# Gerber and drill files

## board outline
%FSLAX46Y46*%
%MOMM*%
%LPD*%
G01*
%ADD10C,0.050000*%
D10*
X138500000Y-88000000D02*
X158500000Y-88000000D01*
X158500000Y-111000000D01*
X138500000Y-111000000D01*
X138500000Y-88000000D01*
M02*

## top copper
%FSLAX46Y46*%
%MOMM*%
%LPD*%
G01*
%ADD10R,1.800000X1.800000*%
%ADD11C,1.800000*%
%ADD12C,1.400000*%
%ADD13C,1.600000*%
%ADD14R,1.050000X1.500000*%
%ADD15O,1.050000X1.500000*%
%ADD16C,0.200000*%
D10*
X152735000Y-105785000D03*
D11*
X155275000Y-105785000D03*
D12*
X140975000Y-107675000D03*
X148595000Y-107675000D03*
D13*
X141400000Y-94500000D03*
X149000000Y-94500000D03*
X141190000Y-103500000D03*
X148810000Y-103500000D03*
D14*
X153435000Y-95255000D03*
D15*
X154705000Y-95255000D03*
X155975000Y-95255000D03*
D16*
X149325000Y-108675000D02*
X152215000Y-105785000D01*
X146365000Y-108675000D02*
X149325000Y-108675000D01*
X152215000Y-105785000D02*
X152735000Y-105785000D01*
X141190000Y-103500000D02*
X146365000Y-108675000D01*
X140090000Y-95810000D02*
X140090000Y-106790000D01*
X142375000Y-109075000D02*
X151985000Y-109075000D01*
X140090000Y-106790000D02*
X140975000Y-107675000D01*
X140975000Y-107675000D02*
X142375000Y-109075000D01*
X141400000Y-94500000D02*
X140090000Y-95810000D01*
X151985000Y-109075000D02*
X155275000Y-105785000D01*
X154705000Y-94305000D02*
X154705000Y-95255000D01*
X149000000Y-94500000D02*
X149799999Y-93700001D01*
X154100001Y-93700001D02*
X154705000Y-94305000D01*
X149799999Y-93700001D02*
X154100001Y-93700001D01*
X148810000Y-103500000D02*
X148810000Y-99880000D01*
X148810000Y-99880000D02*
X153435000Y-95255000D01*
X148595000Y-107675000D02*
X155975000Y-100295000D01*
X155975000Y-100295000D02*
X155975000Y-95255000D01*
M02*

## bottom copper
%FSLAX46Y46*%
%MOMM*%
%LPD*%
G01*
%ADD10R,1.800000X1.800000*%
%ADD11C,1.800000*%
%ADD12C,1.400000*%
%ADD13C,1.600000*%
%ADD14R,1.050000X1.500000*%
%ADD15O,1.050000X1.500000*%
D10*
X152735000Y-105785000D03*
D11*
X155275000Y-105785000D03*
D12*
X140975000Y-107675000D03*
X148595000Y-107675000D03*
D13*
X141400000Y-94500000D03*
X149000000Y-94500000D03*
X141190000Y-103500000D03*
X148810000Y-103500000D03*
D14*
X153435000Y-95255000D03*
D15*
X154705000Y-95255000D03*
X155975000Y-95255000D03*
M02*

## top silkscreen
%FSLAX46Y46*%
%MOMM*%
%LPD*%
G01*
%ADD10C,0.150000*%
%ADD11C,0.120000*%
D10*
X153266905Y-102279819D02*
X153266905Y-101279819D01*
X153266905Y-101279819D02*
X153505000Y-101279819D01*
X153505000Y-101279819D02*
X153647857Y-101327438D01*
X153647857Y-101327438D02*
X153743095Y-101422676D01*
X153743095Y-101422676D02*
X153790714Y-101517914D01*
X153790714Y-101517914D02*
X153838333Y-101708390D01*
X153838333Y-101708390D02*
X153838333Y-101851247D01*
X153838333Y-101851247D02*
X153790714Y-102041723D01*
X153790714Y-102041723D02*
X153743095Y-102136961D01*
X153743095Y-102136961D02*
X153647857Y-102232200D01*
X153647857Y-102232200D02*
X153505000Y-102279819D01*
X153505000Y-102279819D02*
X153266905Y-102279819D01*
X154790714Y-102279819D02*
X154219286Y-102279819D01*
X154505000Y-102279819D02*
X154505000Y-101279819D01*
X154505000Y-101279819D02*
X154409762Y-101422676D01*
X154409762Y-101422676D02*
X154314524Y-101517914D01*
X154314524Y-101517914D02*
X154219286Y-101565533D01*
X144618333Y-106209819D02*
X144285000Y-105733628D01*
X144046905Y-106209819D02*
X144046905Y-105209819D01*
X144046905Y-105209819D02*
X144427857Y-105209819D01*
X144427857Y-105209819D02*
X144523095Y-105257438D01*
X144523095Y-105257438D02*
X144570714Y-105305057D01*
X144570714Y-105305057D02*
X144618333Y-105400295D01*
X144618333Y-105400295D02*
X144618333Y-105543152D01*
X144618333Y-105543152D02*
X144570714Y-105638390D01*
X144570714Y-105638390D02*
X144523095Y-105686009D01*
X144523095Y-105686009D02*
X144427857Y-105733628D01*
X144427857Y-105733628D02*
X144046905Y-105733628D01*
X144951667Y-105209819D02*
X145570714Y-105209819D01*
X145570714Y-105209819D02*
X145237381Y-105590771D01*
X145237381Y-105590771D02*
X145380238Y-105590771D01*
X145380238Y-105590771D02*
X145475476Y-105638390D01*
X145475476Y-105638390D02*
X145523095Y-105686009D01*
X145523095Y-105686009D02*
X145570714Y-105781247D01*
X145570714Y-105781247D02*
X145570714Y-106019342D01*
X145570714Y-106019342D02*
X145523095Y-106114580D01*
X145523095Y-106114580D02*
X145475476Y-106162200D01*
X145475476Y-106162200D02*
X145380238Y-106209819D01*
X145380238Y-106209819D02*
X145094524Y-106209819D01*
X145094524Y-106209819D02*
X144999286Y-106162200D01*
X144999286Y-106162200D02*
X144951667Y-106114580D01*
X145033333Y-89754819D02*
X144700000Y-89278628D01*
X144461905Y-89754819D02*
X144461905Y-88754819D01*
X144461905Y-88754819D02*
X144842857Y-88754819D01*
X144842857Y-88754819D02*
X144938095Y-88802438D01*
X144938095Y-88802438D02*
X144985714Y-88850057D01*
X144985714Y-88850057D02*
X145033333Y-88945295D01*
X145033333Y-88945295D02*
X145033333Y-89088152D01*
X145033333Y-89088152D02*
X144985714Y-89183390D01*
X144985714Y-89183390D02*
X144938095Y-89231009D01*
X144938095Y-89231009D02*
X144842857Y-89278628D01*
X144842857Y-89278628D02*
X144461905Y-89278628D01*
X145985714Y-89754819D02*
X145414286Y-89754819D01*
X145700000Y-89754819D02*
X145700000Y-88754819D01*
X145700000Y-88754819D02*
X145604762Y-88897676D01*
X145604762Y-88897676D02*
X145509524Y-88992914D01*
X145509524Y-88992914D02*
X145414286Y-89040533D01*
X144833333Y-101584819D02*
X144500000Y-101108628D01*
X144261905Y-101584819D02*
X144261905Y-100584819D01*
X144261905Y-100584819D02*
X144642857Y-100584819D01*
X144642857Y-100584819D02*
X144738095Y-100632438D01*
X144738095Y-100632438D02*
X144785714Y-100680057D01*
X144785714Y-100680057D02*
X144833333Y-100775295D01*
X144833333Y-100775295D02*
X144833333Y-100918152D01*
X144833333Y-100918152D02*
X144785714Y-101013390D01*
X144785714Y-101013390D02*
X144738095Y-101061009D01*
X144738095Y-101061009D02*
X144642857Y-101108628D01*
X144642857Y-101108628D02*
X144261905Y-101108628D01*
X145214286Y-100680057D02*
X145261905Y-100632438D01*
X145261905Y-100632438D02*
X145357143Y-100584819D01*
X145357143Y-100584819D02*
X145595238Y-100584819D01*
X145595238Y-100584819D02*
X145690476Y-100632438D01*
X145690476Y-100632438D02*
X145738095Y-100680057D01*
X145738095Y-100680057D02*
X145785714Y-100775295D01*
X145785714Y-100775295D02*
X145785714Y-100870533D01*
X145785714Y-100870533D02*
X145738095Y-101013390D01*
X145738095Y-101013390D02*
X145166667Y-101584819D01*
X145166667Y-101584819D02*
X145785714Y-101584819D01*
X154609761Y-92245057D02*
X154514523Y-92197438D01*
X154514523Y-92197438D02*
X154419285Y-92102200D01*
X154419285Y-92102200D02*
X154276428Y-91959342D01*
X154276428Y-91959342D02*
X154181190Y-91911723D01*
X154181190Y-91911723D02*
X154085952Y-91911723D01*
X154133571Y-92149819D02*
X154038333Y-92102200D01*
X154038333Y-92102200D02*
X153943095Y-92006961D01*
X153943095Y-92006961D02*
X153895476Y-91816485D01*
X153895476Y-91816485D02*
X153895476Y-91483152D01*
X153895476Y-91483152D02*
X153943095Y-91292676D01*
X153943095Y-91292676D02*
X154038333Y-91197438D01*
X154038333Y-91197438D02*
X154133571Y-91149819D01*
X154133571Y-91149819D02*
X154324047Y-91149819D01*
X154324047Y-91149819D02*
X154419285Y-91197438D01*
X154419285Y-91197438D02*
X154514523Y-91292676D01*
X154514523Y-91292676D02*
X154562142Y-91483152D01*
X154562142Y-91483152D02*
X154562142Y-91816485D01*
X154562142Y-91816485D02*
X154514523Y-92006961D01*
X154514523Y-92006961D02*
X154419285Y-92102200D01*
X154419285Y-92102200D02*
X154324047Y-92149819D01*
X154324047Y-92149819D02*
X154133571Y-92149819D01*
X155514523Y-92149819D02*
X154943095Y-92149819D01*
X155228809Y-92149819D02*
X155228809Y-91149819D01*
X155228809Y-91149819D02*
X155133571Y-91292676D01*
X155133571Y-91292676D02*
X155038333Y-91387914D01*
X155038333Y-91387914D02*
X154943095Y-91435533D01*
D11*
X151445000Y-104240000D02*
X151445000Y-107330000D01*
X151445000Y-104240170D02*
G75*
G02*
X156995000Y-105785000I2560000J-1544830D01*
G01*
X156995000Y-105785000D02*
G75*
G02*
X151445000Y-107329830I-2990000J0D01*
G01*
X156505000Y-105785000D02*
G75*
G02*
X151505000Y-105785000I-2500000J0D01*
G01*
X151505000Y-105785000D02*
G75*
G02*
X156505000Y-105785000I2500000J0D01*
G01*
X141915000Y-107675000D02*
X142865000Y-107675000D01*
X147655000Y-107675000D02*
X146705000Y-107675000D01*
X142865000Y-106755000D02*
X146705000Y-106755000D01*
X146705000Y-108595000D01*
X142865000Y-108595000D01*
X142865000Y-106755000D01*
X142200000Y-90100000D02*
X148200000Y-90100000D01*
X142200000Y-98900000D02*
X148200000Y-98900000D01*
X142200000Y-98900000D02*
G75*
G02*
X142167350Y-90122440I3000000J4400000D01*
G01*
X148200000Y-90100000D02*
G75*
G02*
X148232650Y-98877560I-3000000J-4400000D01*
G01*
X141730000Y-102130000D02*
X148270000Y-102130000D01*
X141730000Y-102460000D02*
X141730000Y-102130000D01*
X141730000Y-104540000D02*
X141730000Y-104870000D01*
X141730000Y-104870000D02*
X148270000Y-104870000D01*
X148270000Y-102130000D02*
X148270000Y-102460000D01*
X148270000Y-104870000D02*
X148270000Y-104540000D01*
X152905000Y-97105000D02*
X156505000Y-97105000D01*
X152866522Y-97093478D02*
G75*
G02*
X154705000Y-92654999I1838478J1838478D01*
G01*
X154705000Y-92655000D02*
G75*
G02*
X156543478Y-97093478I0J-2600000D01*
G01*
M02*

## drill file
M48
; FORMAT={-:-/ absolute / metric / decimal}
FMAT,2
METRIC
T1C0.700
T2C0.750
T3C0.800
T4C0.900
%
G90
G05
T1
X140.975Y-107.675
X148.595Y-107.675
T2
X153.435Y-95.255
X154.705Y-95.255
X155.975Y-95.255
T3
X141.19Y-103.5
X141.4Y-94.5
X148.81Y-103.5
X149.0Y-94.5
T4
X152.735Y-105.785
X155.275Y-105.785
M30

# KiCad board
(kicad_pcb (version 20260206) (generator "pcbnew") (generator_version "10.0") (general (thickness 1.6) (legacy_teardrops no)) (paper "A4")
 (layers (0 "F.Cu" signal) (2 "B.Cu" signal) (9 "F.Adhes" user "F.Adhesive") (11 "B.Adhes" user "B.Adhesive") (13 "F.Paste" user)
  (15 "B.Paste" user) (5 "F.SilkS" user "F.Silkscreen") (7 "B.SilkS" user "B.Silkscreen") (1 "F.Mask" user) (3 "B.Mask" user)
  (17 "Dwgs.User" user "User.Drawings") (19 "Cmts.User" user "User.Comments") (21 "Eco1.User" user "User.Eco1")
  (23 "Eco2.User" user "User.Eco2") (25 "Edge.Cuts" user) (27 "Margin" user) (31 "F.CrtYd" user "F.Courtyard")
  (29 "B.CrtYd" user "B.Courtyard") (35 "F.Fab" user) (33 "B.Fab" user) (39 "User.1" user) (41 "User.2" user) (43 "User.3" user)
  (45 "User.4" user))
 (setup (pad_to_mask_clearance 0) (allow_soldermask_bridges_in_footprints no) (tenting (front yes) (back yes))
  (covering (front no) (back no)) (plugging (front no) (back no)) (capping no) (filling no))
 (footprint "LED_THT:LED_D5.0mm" (layer "F.Cu") (at 152.735 105.785)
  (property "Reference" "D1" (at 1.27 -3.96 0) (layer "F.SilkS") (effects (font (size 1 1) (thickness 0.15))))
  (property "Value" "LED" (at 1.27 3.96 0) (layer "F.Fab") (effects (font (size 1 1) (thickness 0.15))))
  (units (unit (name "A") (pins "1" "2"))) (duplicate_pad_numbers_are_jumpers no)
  (fp_line (start -1.29 -1.545) (end -1.29 1.545) (stroke (width 0.12) (type solid)) (layer "F.SilkS"))
  (fp_arc (start -1.29 -1.54483) (mid 2.071779 -2.880495) (end 4.26 0) (stroke (width 0.12) (type solid)) (layer "F.SilkS"))
  (fp_arc (start 4.26 0) (mid 2.071779 2.880495) (end -1.29 1.54483) (stroke (width 0.12) (type solid)) (layer "F.SilkS"))
  (fp_circle (center 1.27 0) (end 3.77 0) (stroke (width 0.12) (type solid)) (fill no) (layer "F.SilkS"))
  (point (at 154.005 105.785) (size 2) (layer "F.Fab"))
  (pad "1" thru_hole rect (at 0 0) (size 1.8 1.8) (drill 0.9) (layers "*.Cu" "*.Mask") (remove_unused_layers no) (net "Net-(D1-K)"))
  (pad "2" thru_hole circle (at 2.54 0) (size 1.8 1.8) (drill 0.9) (layers "*.Cu" "*.Mask") (remove_unused_layers no) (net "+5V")))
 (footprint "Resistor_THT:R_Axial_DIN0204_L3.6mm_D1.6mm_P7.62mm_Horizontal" (layer "F.Cu") (at 140.975 107.675)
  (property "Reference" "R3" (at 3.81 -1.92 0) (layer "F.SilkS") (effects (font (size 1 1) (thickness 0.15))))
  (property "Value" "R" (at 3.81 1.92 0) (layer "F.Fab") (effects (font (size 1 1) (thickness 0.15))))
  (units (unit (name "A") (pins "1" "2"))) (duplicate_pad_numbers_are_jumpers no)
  (fp_line (start 0.94 0) (end 1.89 0) (stroke (width 0.12) (type solid)) (layer "F.SilkS"))
  (fp_line (start 6.68 0) (end 5.73 0) (stroke (width 0.12) (type solid)) (layer "F.SilkS"))
  (fp_rect (start 1.89 -0.92) (end 5.73 0.92) (stroke (width 0.12) (type solid)) (fill no) (layer "F.SilkS"))
  (pad "1" thru_hole circle (at 0 0) (size 1.4 1.4) (drill 0.7) (layers "*.Cu" "*.Mask") (remove_unused_layers no) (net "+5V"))
  (pad "2" thru_hole circle (at 7.62 0) (size 1.4 1.4) (drill 0.7) (layers "*.Cu" "*.Mask") (remove_unused_layers no) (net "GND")))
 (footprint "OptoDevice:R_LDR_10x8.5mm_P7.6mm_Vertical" (layer "F.Cu") (at 141.4 94.5)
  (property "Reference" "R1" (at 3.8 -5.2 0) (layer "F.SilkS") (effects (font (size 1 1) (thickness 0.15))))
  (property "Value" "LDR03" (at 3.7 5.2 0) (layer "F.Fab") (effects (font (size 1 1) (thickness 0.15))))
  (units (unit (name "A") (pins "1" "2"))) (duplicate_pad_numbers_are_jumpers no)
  (fp_line (start 0.8 -4.4) (end 6.8 -4.4) (stroke (width 0.12) (type solid)) (layer "F.SilkS"))
  (fp_line (start 0.8 4.4) (end 6.8 4.4) (stroke (width 0.12) (type solid)) (layer "F.SilkS"))
  (fp_arc (start 0.8 4.4) (mid -1.525374 0.019809) (end 0.76735 -4.37756) (stroke (width 0.12) (type solid)) (layer "F.SilkS"))
  (fp_arc (start 6.8 -4.4) (mid 9.125374 -0.019809) (end 6.83265 4.37756) (stroke (width 0.12) (type solid)) (layer "F.SilkS"))
  (pad "1" thru_hole circle (at 0 0) (size 1.6 1.6) (drill 0.8) (layers "*.Cu" "*.Mask") (remove_unused_layers no) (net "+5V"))
  (pad "2" thru_hole circle (at 7.6 0) (size 1.6 1.6) (drill 0.8) (layers "*.Cu" "*.Mask") (remove_unused_layers no) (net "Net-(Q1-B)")))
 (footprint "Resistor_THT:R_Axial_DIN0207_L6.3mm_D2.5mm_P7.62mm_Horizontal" (layer "F.Cu") (at 141.19 103.5)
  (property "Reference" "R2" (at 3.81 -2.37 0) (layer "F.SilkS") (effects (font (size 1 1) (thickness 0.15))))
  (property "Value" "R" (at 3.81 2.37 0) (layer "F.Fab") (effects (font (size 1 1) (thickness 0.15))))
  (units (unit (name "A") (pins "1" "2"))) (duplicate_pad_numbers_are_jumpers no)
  (fp_line (start 0.54 -1.37) (end 7.08 -1.37) (stroke (width 0.12) (type solid)) (layer "F.SilkS"))
  (fp_line (start 0.54 -1.04) (end 0.54 -1.37) (stroke (width 0.12) (type solid)) (layer "F.SilkS"))
  (fp_line (start 0.54 1.04) (end 0.54 1.37) (stroke (width 0.12) (type solid)) (layer "F.SilkS"))
  (fp_line (start 0.54 1.37) (end 7.08 1.37) (stroke (width 0.12) (type solid)) (layer "F.SilkS"))
  (fp_line (start 7.08 -1.37) (end 7.08 -1.04) (stroke (width 0.12) (type solid)) (layer "F.SilkS"))
  (fp_line (start 7.08 1.37) (end 7.08 1.04) (stroke (width 0.12) (type solid)) (layer "F.SilkS"))
  (pad "1" thru_hole circle (at 0 0) (size 1.6 1.6) (drill 0.8) (layers "*.Cu" "*.Mask") (remove_unused_layers no) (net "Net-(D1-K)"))
  (pad "2" thru_hole circle (at 7.62 0) (size 1.6 1.6) (drill 0.8) (layers "*.Cu" "*.Mask") (remove_unused_layers no) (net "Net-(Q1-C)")))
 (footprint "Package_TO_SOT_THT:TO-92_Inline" (layer "F.Cu") (at 153.435 95.255)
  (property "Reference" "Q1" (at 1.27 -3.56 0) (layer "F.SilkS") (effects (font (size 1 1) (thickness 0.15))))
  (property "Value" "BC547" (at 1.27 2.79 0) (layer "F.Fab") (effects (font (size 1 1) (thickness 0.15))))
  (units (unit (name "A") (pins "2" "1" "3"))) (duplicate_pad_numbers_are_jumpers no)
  (fp_line (start -0.53 1.85) (end 3.07 1.85) (stroke (width 0.12) (type solid)) (layer "F.SilkS"))
  (fp_arc (start -0.568478 1.838478) (mid -1.132087 -0.994977) (end 1.27 -2.6) (stroke (width 0.12) (type solid)) (layer "F.SilkS"))
  (fp_arc (start 1.27 -2.6) (mid 3.672087 -0.994977) (end 3.108478 1.838478) (stroke (width 0.12) (type solid)) (layer "F.SilkS"))
  (pad "1" thru_hole rect (at 0 0) (size 1.05 1.5) (drill 0.75) (layers "*.Cu" "*.Mask") (remove_unused_layers no) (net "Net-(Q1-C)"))
  (pad "2" thru_hole oval (at 1.27 0) (size 1.05 1.5) (drill 0.75) (layers "*.Cu" "*.Mask") (remove_unused_layers no) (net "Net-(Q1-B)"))
  (pad "3" thru_hole oval (at 2.54 0) (size 1.05 1.5) (drill 0.75) (layers "*.Cu" "*.Mask") (remove_unused_layers no) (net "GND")))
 (gr_rect (start 138.5 88) (end 158.5 111) (stroke (width 0.05) (type default)) (fill no) (layer "Edge.Cuts"))
 (segment (start 149.325 108.675) (end 152.215 105.785) (width 0.2) (layer "F.Cu") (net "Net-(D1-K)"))
 (segment (start 146.365 108.675) (end 149.325 108.675) (width 0.2) (layer "F.Cu") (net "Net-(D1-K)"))
 (segment (start 152.215 105.785) (end 152.735 105.785) (width 0.2) (layer "F.Cu") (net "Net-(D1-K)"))
 (segment (start 141.19 103.5) (end 146.365 108.675) (width 0.2) (layer "F.Cu") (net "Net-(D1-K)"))
 (segment (start 140.09 95.81) (end 140.09 106.79) (width 0.2) (layer "F.Cu") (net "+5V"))
 (segment (start 142.375 109.075) (end 151.985 109.075) (width 0.2) (layer "F.Cu") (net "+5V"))
 (segment (start 140.09 106.79) (end 140.975 107.675) (width 0.2) (layer "F.Cu") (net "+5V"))
 (segment (start 140.975 107.675) (end 142.375 109.075) (width 0.2) (layer "F.Cu") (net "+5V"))
 (segment (start 141.4 94.5) (end 140.09 95.81) (width 0.2) (layer "F.Cu") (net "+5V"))
 (segment (start 151.985 109.075) (end 155.275 105.785) (width 0.2) (layer "F.Cu") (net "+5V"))
 (segment (start 154.705 94.305) (end 154.705 95.255) (width 0.2) (layer "F.Cu") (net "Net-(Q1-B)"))
 (segment (start 149 94.5) (end 149.799999 93.700001) (width 0.2) (layer "F.Cu") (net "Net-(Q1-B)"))
 (segment (start 154.100001 93.700001) (end 154.705 94.305) (width 0.2) (layer "F.Cu") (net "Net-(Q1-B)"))
 (segment (start 149.799999 93.700001) (end 154.100001 93.700001) (width 0.2) (layer "F.Cu") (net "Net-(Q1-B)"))
 (segment (start 148.81 103.5) (end 148.81 99.88) (width 0.2) (layer "F.Cu") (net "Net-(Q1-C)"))
 (segment (start 148.81 99.88) (end 153.435 95.255) (width 0.2) (layer "F.Cu") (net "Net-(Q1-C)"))
 (segment (start 148.595 107.675) (end 155.975 100.295) (width 0.2) (layer "F.Cu") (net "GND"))
 (segment (start 155.975 100.295) (end 155.975 95.255) (width 0.2) (layer "F.Cu") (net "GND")))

